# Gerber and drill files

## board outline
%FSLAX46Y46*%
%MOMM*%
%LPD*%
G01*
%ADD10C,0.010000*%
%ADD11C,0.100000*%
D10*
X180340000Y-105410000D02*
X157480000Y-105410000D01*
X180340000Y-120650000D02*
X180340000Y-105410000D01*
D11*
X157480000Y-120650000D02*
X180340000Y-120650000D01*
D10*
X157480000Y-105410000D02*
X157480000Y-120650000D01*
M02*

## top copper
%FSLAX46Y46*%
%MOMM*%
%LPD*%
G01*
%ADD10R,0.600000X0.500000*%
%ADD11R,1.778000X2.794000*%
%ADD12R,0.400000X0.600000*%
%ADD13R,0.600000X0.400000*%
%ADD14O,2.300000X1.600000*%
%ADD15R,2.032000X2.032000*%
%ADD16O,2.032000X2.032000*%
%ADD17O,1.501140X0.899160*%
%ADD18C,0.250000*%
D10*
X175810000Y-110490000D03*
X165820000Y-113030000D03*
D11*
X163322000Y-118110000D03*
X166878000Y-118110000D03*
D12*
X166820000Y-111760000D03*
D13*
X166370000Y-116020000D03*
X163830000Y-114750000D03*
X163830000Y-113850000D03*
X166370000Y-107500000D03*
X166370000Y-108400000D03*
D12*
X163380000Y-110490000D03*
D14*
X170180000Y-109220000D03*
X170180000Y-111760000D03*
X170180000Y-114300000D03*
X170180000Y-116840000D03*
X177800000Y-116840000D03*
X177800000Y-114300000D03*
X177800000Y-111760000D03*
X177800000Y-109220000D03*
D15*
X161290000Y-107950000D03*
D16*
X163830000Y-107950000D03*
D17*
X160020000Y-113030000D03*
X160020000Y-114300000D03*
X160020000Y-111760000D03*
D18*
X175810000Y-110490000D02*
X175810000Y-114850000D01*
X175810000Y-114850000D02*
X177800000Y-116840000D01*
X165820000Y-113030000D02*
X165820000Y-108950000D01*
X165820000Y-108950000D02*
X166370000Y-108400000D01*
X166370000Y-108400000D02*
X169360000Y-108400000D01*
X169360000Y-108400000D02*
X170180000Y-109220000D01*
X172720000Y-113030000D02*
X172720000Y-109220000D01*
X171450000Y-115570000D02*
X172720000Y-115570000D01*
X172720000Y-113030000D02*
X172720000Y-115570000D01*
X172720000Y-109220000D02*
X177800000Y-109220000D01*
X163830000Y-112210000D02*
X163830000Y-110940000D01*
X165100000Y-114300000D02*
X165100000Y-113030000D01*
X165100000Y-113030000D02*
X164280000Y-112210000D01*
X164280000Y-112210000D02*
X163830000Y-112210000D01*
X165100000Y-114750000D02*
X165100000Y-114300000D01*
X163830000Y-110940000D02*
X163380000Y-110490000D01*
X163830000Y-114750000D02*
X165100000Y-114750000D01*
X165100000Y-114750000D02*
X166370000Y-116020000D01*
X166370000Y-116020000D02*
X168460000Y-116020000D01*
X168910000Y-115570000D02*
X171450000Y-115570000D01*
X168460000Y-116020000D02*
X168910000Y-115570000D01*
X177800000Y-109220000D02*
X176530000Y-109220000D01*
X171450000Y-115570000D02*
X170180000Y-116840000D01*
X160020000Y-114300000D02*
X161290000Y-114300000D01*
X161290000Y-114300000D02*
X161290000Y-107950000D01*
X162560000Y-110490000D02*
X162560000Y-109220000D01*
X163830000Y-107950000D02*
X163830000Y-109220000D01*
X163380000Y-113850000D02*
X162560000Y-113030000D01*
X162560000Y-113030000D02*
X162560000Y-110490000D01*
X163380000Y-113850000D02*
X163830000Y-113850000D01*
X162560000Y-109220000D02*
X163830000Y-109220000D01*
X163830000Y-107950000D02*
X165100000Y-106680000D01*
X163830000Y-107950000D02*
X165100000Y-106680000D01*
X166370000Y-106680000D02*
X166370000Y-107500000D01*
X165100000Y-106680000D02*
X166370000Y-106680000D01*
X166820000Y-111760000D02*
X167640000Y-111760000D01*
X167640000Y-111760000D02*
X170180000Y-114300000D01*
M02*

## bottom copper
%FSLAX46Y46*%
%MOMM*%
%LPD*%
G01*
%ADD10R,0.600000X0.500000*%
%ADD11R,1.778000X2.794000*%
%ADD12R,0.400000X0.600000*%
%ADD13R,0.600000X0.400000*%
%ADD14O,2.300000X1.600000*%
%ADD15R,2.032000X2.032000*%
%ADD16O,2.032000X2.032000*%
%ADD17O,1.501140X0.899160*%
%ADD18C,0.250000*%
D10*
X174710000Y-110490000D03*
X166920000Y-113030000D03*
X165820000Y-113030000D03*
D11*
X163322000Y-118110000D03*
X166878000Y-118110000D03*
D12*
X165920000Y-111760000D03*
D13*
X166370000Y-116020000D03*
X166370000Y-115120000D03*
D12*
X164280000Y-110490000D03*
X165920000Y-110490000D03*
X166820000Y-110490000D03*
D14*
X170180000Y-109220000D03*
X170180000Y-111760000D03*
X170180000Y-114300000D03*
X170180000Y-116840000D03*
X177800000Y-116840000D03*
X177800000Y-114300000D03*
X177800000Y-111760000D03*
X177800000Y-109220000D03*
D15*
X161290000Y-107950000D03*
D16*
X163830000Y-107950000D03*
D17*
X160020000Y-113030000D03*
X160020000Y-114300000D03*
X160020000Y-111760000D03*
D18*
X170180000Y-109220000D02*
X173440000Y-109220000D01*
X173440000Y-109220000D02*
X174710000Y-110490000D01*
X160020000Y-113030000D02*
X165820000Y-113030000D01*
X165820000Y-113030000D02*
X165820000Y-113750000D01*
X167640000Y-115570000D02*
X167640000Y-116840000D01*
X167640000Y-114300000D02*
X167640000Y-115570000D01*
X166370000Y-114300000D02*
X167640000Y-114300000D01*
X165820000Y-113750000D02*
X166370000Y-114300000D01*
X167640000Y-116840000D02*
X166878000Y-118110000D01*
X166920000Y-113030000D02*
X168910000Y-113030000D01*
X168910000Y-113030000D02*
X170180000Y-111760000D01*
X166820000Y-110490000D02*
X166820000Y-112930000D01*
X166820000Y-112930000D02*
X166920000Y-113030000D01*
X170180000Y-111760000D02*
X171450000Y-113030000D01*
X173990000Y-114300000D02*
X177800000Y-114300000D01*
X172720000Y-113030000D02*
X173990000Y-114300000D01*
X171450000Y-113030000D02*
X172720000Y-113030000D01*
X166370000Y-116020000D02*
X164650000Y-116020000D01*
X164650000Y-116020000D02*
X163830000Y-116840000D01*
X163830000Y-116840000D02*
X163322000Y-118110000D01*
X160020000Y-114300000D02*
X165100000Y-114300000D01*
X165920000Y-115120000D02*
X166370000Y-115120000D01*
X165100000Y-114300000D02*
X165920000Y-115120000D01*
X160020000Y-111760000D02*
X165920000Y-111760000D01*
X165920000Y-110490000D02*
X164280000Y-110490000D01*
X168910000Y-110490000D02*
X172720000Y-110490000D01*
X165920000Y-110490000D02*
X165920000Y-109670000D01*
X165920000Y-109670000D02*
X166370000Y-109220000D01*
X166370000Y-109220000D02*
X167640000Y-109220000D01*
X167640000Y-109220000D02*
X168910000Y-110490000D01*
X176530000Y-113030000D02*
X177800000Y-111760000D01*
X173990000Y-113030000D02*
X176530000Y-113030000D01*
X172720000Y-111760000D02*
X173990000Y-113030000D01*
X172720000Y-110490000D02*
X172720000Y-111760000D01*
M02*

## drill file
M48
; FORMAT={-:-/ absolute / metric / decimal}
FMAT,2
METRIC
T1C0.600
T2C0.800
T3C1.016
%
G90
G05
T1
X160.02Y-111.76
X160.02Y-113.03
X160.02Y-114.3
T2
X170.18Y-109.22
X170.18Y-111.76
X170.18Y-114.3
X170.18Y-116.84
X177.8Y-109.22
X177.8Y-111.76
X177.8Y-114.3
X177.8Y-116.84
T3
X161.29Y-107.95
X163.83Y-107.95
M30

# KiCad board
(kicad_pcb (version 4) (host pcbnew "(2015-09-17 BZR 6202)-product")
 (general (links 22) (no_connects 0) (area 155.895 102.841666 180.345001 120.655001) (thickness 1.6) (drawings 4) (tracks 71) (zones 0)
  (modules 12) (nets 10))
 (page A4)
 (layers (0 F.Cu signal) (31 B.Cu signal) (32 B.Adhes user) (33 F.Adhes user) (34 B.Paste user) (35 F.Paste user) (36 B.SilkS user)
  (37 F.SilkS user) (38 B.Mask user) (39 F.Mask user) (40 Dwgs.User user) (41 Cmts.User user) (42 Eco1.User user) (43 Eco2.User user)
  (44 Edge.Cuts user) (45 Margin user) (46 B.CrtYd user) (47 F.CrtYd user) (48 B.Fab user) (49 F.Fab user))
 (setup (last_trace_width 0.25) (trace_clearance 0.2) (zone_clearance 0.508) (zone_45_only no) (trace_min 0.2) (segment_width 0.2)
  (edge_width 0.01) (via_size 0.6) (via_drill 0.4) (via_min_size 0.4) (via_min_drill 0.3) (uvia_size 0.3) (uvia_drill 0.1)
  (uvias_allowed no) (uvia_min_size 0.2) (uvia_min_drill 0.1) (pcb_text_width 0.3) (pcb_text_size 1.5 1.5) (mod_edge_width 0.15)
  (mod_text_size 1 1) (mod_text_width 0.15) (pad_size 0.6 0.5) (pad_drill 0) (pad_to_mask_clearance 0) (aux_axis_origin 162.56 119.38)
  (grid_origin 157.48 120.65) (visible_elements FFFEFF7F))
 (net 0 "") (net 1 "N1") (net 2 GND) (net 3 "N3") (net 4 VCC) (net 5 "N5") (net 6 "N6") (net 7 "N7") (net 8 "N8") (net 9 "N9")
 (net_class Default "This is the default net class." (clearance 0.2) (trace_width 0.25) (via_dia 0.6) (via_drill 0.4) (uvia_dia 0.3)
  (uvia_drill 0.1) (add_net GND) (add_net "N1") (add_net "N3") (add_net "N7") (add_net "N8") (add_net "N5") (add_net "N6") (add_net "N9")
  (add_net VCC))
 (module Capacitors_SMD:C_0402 (layer B.Cu) (at 175.26 110.49 180)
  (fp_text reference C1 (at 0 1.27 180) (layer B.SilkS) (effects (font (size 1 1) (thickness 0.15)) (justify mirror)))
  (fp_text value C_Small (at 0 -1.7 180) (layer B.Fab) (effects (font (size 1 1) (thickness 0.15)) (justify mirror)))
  (pad 1 smd rect (at -0.55 0 180) (size 0.6 0.5) (layers F.Cu B.Paste B.Mask) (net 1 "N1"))
  (pad 2 smd rect (at 0.55 0 180) (size 0.6 0.5) (layers B.Cu B.Paste B.Mask) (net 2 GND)))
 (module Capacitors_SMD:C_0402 (layer F.Cu) (at 166.37 113.03 180)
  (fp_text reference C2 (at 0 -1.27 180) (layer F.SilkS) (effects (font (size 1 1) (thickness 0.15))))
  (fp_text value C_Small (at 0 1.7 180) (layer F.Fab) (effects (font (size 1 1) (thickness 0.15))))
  (pad 1 smd rect (at -0.55 0 180) (size 0.6 0.5) (layers B.Cu F.Paste F.Mask) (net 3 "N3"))
  (pad 2 smd rect (at 0.55 0 180) (size 0.6 0.5) (layers *.Cu F.Paste F.Mask) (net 2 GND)))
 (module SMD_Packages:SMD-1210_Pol (layer F.Cu) (at 165.1 118.11)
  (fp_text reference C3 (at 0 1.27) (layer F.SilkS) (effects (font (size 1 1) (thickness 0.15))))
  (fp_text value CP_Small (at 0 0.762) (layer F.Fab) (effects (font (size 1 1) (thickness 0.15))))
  (pad 1 smd rect (at -1.778 0) (size 1.778 2.794) (layers *.Cu F.Paste F.Mask) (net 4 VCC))
  (pad 2 smd rect (at 1.778 0) (size 1.778 2.794) (layers *.Cu F.Paste F.Mask) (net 2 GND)))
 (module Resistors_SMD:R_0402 (layer F.Cu) (at 166.37 111.76)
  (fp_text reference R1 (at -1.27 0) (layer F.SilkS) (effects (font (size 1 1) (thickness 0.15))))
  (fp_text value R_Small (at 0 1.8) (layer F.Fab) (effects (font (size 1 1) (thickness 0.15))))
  (pad 1 smd rect (at -0.45 0) (size 0.4 0.6) (layers B.Cu F.Paste F.Mask) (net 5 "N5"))
  (pad 2 smd rect (at 0.45 0) (size 0.4 0.6) (layers F.Cu F.Paste F.Mask) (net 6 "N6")))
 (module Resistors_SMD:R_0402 (layer F.Cu) (at 166.37 115.57 90)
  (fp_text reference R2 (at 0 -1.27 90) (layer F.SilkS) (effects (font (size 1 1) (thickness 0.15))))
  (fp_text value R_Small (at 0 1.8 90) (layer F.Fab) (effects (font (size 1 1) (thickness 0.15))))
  (pad 1 smd rect (at -0.45 0 90) (size 0.4 0.6) (layers *.Cu F.Paste F.Mask) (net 4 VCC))
  (pad 2 smd rect (at 0.45 0 90) (size 0.4 0.6) (layers B.Cu F.Paste F.Mask) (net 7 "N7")))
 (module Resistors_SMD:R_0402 (layer F.Cu) (at 163.83 114.3 90)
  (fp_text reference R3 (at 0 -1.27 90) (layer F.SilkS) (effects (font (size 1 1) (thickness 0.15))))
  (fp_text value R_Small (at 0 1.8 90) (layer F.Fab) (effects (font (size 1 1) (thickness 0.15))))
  (pad 1 smd rect (at -0.45 0 90) (size 0.4 0.6) (layers F.Cu F.Paste F.Mask) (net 4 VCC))
  (pad 2 smd rect (at 0.45 0 90) (size 0.4 0.6) (layers F.Cu F.Paste F.Mask) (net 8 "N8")))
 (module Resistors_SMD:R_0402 (layer F.Cu) (at 166.37 107.95 270)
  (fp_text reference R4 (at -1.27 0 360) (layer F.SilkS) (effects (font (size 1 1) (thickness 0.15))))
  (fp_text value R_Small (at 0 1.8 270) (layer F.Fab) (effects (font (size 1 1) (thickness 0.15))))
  (pad 1 smd rect (at -0.45 0 270) (size 0.4 0.6) (layers F.Cu F.Paste F.Mask) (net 8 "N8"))
  (pad 2 smd rect (at 0.45 0 270) (size 0.4 0.6) (layers F.Cu F.Paste F.Mask) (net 2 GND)))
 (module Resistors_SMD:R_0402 (layer F.Cu) (at 163.83 110.49)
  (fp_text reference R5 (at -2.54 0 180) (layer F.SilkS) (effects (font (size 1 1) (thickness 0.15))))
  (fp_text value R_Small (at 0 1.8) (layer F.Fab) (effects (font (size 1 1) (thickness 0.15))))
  (pad 1 smd rect (at -0.45 0) (size 0.4 0.6) (layers F.Cu F.Paste F.Mask) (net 4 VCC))
  (pad 2 smd rect (at 0.45 0) (size 0.4 0.6) (layers B.Cu F.Paste F.Mask) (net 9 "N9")))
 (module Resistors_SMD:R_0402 (layer F.Cu) (at 166.37 110.49)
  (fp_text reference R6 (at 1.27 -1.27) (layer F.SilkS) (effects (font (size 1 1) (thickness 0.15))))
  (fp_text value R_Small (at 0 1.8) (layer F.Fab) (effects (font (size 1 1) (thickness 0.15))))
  (pad 1 smd rect (at -0.45 0) (size 0.4 0.6) (layers B.Cu F.Paste F.Mask) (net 9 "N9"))
  (pad 2 smd rect (at 0.45 0) (size 0.4 0.6) (layers B.Cu F.Paste F.Mask) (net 3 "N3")))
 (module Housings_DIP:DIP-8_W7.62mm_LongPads (layer F.Cu) (at 170.18 109.22)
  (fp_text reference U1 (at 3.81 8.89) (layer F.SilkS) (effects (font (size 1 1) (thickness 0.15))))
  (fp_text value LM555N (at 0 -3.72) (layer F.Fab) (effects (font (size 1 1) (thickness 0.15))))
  (pad 1 thru_hole oval (at 0 0) (size 2.3 1.6) (drill 0.8) (layers *.Cu *.Mask F.SilkS) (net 2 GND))
  (pad 2 thru_hole oval (at 0 2.54) (size 2.3 1.6) (drill 0.8) (layers *.Cu *.Mask F.SilkS) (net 3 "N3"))
  (pad 3 thru_hole oval (at 0 5.08) (size 2.3 1.6) (drill 0.8) (layers *.Cu *.Mask F.SilkS) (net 6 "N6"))
  (pad 4 thru_hole oval (at 0 7.62) (size 2.3 1.6) (drill 0.8) (layers *.Cu *.Mask F.SilkS) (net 4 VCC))
  (pad 5 thru_hole oval (at 7.62 7.62) (size 2.3 1.6) (drill 0.8) (layers *.Cu *.Mask F.SilkS) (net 1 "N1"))
  (pad 6 thru_hole oval (at 7.62 5.08) (size 2.3 1.6) (drill 0.8) (layers *.Cu *.Mask F.SilkS) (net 3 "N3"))
  (pad 7 thru_hole oval (at 7.62 2.54) (size 2.3 1.6) (drill 0.8) (layers *.Cu *.Mask F.SilkS) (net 9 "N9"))
  (pad 8 thru_hole oval (at 7.62 0) (size 2.3 1.6) (drill 0.8) (layers *.Cu *.Mask F.SilkS) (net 4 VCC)))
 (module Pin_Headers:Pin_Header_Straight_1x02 (layer F.Cu) (at 161.29 107.95 90)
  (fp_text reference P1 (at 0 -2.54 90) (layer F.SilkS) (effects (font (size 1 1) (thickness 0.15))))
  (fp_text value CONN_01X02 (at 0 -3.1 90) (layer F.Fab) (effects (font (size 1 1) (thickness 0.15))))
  (pad 1 thru_hole rect (at 0 0 90) (size 2.032 2.032) (drill 1.016) (layers *.Cu *.Mask F.SilkS) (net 7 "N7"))
  (pad 2 thru_hole oval (at 0 2.54 90) (size 2.032 2.032) (drill 1.016) (layers *.Cu *.Mask F.SilkS) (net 8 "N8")))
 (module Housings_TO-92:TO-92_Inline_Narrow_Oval (layer F.Cu) (at 160.02 111.76 270)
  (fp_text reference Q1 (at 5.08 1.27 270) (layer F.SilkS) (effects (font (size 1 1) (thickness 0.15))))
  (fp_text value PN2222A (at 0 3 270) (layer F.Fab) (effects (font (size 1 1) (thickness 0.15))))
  (pad 2 thru_hole oval (at 1.27 0 90) (size 0.89916 1.50114) (drill 0.6) (layers *.Cu *.Mask F.SilkS) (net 2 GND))
  (pad 3 thru_hole oval (at 2.54 0 90) (size 0.89916 1.50114) (drill 0.6) (layers *.Cu *.Mask F.SilkS) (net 7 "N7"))
  (pad 1 thru_hole oval (at 0 0 90) (size 0.89916 1.50114) (drill 0.6) (layers *.Cu *.Mask F.SilkS) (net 5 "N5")))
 (gr_line (start 180.34 105.41) (end 157.48 105.41) (angle 90) (layer Edge.Cuts) (width 0.01))
 (gr_line (start 180.34 120.65) (end 180.34 105.41) (angle 90) (layer Edge.Cuts) (width 0.01))
 (gr_line (start 157.48 120.65) (end 180.34 120.65) (angle 90) (layer Edge.Cuts) (width 0.1))
 (gr_line (start 157.48 105.41) (end 157.48 120.65) (angle 90) (layer Edge.Cuts) (width 0.01))
 (segment (start 175.81 110.49) (end 175.81 114.85) (width 0.25) (layer F.Cu) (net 1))
 (segment (start 175.81 114.85) (end 177.8 116.84) (width 0.25) (layer F.Cu) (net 1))
 (segment (start 170.18 109.22) (end 173.44 109.22) (width 0.25) (layer B.Cu) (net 2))
 (segment (start 173.44 109.22) (end 174.71 110.49) (width 0.25) (layer B.Cu) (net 2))
 (segment (start 160.02 113.03) (end 165.82 113.03) (width 0.25) (layer B.Cu) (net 2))
 (segment (start 165.82 113.03) (end 165.82 113.75) (width 0.25) (layer B.Cu) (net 2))
 (segment (start 167.64 115.57) (end 167.64 116.84) (width 0.25) (layer B.Cu) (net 2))
 (segment (start 167.64 114.3) (end 167.64 115.57) (width 0.25) (layer B.Cu) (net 2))
 (segment (start 166.37 114.3) (end 167.64 114.3) (width 0.25) (layer B.Cu) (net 2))
 (segment (start 165.82 113.75) (end 166.37 114.3) (width 0.25) (layer B.Cu) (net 2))
 (segment (start 167.64 116.84) (end 166.878 118.11) (width 0.25) (layer B.Cu) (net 2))
 (segment (start 165.82 113.03) (end 165.82 108.95) (width 0.25) (layer F.Cu) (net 2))
 (segment (start 165.82 108.95) (end 166.37 108.4) (width 0.25) (layer F.Cu) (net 2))
 (segment (start 166.37 108.4) (end 169.36 108.4) (width 0.25) (layer F.Cu) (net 2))
 (segment (start 169.36 108.4) (end 170.18 109.22) (width 0.25) (layer F.Cu) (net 2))
 (segment (start 166.92 113.03) (end 168.91 113.03) (width 0.25) (layer B.Cu) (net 3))
 (segment (start 168.91 113.03) (end 170.18 111.76) (width 0.25) (layer B.Cu) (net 3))
 (segment (start 166.82 110.49) (end 166.82 112.93) (width 0.25) (layer B.Cu) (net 3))
 (segment (start 166.82 112.93) (end 166.92 113.03) (width 0.25) (layer B.Cu) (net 3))
 (segment (start 170.18 111.76) (end 171.45 113.03) (width 0.25) (layer B.Cu) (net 3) (status 80000))
 (segment (start 173.99 114.3) (end 177.8 114.3) (width 0.25) (layer B.Cu) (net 3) (status 80000))
 (segment (start 172.72 113.03) (end 173.99 114.3) (width 0.25) (layer B.Cu) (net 3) (status 80000))
 (segment (start 171.45 113.03) (end 172.72 113.03) (width 0.25) (layer B.Cu) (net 3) (status 80000))
 (segment (start 172.72 113.03) (end 172.72 109.22) (width 0.25) (layer F.Cu) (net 4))
 (segment (start 171.45 115.57) (end 172.72 115.57) (width 0.25) (layer F.Cu) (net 4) (status 80000))
 (segment (start 172.72 113.03) (end 172.72 115.57) (width 0.25) (layer F.Cu) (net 4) (status 80000))
 (segment (start 172.72 109.22) (end 177.8 109.22) (width 0.25) (layer F.Cu) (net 4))
 (segment (start 163.83 112.21) (end 163.83 110.94) (width 0.25) (layer F.Cu) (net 4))
 (segment (start 165.1 114.3) (end 165.1 113.03) (width 0.25) (layer F.Cu) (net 4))
 (segment (start 165.1 113.03) (end 164.28 112.21) (width 0.25) (layer F.Cu) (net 4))
 (segment (start 164.28 112.21) (end 163.83 112.21) (width 0.25) (layer F.Cu) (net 4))
 (segment (start 165.1 114.75) (end 165.1 114.3) (width 0.25) (layer F.Cu) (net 4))
 (segment (start 163.83 110.94) (end 163.38 110.49) (width 0.25) (layer F.Cu) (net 4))
 (segment (start 163.83 114.75) (end 165.1 114.75) (width 0.25) (layer F.Cu) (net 4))
 (segment (start 165.1 114.75) (end 166.37 116.02) (width 0.25) (layer F.Cu) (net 4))
 (segment (start 166.37 116.02) (end 164.65 116.02) (width 0.25) (layer B.Cu) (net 4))
 (segment (start 164.65 116.02) (end 163.83 116.84) (width 0.25) (layer B.Cu) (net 4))
 (segment (start 163.83 116.84) (end 163.322 118.11) (width 0.25) (layer B.Cu) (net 4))
 (segment (start 166.37 116.02) (end 168.46 116.02) (width 0.25) (layer F.Cu) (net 4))
 (segment (start 168.91 115.57) (end 171.45 115.57) (width 0.25) (layer F.Cu) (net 4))
 (segment (start 168.46 116.02) (end 168.91 115.57) (width 0.25) (layer F.Cu) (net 4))
 (segment (start 177.8 109.22) (end 176.53 109.22) (width 0.25) (layer F.Cu) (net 4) (status 80000))
 (segment (start 171.45 115.57) (end 170.18 116.84) (width 0.25) (layer F.Cu) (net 4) (status 80000))
 (segment (start 160.02 114.3) (end 161.29 114.3) (width 0.25) (layer F.Cu) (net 7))
 (segment (start 161.29 114.3) (end 161.29 107.95) (width 0.25) (layer F.Cu) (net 7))
 (segment (start 160.02 114.3) (end 165.1 114.3) (width 0.25) (layer B.Cu) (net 7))
 (segment (start 165.92 115.12) (end 166.37 115.12) (width 0.25) (layer B.Cu) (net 7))
 (segment (start 165.1 114.3) (end 165.92 115.12) (width 0.25) (layer B.Cu) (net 7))
 (segment (start 162.56 110.49) (end 162.56 109.22) (width 0.25) (layer F.Cu) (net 8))
 (segment (start 163.83 107.95) (end 163.83 109.22) (width 0.25) (layer F.Cu) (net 8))
 (segment (start 163.38 113.85) (end 162.56 113.03) (width 0.25) (layer F.Cu) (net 8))
 (segment (start 162.56 113.03) (end 162.56 110.49) (width 0.25) (layer F.Cu) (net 8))
 (segment (start 163.38 113.85) (end 163.83 113.85) (width 0.25) (layer F.Cu) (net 8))
 (segment (start 162.56 109.22) (end 163.83 109.22) (width 0.25) (layer F.Cu) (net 8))
 (segment (start 163.83 107.95) (end 165.1 106.68) (width 0.25) (layer F.Cu) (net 8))
 (segment (start 163.83 107.95) (end 165.1 106.68) (width 0.25) (layer F.Cu) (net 8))
 (segment (start 166.37 106.68) (end 166.37 107.5) (width 0.25) (layer F.Cu) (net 8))
 (segment (start 165.1 106.68) (end 166.37 106.68) (width 0.25) (layer F.Cu) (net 8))
 (segment (start 160.02 111.76) (end 165.92 111.76) (width 0.25) (layer B.Cu) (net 5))
 (segment (start 166.82 111.76) (end 167.64 111.76) (width 0.25) (layer F.Cu) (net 6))
 (segment (start 167.64 111.76) (end 170.18 114.3) (width 0.25) (layer F.Cu) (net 6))
 (segment (start 165.92 110.49) (end 164.28 110.49) (width 0.25) (layer B.Cu) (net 9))
 (segment (start 168.91 110.49) (end 172.72 110.49) (width 0.25) (layer B.Cu) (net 9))
 (segment (start 165.92 110.49) (end 165.92 109.67) (width 0.25) (layer B.Cu) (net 9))
 (segment (start 165.92 109.67) (end 166.37 109.22) (width 0.25) (layer B.Cu) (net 9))
 (segment (start 166.37 109.22) (end 167.64 109.22) (width 0.25) (layer B.Cu) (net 9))
 (segment (start 167.64 109.22) (end 168.91 110.49) (width 0.25) (layer B.Cu) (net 9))
 (segment (start 176.53 113.03) (end 177.8 111.76) (width 0.25) (layer B.Cu) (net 9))
 (segment (start 173.99 113.03) (end 176.53 113.03) (width 0.25) (layer B.Cu) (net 9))
 (segment (start 172.72 111.76) (end 173.99 113.03) (width 0.25) (layer B.Cu) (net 9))
 (segment (start 172.72 110.49) (end 172.72 111.76) (width 0.25) (layer B.Cu) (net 9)))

